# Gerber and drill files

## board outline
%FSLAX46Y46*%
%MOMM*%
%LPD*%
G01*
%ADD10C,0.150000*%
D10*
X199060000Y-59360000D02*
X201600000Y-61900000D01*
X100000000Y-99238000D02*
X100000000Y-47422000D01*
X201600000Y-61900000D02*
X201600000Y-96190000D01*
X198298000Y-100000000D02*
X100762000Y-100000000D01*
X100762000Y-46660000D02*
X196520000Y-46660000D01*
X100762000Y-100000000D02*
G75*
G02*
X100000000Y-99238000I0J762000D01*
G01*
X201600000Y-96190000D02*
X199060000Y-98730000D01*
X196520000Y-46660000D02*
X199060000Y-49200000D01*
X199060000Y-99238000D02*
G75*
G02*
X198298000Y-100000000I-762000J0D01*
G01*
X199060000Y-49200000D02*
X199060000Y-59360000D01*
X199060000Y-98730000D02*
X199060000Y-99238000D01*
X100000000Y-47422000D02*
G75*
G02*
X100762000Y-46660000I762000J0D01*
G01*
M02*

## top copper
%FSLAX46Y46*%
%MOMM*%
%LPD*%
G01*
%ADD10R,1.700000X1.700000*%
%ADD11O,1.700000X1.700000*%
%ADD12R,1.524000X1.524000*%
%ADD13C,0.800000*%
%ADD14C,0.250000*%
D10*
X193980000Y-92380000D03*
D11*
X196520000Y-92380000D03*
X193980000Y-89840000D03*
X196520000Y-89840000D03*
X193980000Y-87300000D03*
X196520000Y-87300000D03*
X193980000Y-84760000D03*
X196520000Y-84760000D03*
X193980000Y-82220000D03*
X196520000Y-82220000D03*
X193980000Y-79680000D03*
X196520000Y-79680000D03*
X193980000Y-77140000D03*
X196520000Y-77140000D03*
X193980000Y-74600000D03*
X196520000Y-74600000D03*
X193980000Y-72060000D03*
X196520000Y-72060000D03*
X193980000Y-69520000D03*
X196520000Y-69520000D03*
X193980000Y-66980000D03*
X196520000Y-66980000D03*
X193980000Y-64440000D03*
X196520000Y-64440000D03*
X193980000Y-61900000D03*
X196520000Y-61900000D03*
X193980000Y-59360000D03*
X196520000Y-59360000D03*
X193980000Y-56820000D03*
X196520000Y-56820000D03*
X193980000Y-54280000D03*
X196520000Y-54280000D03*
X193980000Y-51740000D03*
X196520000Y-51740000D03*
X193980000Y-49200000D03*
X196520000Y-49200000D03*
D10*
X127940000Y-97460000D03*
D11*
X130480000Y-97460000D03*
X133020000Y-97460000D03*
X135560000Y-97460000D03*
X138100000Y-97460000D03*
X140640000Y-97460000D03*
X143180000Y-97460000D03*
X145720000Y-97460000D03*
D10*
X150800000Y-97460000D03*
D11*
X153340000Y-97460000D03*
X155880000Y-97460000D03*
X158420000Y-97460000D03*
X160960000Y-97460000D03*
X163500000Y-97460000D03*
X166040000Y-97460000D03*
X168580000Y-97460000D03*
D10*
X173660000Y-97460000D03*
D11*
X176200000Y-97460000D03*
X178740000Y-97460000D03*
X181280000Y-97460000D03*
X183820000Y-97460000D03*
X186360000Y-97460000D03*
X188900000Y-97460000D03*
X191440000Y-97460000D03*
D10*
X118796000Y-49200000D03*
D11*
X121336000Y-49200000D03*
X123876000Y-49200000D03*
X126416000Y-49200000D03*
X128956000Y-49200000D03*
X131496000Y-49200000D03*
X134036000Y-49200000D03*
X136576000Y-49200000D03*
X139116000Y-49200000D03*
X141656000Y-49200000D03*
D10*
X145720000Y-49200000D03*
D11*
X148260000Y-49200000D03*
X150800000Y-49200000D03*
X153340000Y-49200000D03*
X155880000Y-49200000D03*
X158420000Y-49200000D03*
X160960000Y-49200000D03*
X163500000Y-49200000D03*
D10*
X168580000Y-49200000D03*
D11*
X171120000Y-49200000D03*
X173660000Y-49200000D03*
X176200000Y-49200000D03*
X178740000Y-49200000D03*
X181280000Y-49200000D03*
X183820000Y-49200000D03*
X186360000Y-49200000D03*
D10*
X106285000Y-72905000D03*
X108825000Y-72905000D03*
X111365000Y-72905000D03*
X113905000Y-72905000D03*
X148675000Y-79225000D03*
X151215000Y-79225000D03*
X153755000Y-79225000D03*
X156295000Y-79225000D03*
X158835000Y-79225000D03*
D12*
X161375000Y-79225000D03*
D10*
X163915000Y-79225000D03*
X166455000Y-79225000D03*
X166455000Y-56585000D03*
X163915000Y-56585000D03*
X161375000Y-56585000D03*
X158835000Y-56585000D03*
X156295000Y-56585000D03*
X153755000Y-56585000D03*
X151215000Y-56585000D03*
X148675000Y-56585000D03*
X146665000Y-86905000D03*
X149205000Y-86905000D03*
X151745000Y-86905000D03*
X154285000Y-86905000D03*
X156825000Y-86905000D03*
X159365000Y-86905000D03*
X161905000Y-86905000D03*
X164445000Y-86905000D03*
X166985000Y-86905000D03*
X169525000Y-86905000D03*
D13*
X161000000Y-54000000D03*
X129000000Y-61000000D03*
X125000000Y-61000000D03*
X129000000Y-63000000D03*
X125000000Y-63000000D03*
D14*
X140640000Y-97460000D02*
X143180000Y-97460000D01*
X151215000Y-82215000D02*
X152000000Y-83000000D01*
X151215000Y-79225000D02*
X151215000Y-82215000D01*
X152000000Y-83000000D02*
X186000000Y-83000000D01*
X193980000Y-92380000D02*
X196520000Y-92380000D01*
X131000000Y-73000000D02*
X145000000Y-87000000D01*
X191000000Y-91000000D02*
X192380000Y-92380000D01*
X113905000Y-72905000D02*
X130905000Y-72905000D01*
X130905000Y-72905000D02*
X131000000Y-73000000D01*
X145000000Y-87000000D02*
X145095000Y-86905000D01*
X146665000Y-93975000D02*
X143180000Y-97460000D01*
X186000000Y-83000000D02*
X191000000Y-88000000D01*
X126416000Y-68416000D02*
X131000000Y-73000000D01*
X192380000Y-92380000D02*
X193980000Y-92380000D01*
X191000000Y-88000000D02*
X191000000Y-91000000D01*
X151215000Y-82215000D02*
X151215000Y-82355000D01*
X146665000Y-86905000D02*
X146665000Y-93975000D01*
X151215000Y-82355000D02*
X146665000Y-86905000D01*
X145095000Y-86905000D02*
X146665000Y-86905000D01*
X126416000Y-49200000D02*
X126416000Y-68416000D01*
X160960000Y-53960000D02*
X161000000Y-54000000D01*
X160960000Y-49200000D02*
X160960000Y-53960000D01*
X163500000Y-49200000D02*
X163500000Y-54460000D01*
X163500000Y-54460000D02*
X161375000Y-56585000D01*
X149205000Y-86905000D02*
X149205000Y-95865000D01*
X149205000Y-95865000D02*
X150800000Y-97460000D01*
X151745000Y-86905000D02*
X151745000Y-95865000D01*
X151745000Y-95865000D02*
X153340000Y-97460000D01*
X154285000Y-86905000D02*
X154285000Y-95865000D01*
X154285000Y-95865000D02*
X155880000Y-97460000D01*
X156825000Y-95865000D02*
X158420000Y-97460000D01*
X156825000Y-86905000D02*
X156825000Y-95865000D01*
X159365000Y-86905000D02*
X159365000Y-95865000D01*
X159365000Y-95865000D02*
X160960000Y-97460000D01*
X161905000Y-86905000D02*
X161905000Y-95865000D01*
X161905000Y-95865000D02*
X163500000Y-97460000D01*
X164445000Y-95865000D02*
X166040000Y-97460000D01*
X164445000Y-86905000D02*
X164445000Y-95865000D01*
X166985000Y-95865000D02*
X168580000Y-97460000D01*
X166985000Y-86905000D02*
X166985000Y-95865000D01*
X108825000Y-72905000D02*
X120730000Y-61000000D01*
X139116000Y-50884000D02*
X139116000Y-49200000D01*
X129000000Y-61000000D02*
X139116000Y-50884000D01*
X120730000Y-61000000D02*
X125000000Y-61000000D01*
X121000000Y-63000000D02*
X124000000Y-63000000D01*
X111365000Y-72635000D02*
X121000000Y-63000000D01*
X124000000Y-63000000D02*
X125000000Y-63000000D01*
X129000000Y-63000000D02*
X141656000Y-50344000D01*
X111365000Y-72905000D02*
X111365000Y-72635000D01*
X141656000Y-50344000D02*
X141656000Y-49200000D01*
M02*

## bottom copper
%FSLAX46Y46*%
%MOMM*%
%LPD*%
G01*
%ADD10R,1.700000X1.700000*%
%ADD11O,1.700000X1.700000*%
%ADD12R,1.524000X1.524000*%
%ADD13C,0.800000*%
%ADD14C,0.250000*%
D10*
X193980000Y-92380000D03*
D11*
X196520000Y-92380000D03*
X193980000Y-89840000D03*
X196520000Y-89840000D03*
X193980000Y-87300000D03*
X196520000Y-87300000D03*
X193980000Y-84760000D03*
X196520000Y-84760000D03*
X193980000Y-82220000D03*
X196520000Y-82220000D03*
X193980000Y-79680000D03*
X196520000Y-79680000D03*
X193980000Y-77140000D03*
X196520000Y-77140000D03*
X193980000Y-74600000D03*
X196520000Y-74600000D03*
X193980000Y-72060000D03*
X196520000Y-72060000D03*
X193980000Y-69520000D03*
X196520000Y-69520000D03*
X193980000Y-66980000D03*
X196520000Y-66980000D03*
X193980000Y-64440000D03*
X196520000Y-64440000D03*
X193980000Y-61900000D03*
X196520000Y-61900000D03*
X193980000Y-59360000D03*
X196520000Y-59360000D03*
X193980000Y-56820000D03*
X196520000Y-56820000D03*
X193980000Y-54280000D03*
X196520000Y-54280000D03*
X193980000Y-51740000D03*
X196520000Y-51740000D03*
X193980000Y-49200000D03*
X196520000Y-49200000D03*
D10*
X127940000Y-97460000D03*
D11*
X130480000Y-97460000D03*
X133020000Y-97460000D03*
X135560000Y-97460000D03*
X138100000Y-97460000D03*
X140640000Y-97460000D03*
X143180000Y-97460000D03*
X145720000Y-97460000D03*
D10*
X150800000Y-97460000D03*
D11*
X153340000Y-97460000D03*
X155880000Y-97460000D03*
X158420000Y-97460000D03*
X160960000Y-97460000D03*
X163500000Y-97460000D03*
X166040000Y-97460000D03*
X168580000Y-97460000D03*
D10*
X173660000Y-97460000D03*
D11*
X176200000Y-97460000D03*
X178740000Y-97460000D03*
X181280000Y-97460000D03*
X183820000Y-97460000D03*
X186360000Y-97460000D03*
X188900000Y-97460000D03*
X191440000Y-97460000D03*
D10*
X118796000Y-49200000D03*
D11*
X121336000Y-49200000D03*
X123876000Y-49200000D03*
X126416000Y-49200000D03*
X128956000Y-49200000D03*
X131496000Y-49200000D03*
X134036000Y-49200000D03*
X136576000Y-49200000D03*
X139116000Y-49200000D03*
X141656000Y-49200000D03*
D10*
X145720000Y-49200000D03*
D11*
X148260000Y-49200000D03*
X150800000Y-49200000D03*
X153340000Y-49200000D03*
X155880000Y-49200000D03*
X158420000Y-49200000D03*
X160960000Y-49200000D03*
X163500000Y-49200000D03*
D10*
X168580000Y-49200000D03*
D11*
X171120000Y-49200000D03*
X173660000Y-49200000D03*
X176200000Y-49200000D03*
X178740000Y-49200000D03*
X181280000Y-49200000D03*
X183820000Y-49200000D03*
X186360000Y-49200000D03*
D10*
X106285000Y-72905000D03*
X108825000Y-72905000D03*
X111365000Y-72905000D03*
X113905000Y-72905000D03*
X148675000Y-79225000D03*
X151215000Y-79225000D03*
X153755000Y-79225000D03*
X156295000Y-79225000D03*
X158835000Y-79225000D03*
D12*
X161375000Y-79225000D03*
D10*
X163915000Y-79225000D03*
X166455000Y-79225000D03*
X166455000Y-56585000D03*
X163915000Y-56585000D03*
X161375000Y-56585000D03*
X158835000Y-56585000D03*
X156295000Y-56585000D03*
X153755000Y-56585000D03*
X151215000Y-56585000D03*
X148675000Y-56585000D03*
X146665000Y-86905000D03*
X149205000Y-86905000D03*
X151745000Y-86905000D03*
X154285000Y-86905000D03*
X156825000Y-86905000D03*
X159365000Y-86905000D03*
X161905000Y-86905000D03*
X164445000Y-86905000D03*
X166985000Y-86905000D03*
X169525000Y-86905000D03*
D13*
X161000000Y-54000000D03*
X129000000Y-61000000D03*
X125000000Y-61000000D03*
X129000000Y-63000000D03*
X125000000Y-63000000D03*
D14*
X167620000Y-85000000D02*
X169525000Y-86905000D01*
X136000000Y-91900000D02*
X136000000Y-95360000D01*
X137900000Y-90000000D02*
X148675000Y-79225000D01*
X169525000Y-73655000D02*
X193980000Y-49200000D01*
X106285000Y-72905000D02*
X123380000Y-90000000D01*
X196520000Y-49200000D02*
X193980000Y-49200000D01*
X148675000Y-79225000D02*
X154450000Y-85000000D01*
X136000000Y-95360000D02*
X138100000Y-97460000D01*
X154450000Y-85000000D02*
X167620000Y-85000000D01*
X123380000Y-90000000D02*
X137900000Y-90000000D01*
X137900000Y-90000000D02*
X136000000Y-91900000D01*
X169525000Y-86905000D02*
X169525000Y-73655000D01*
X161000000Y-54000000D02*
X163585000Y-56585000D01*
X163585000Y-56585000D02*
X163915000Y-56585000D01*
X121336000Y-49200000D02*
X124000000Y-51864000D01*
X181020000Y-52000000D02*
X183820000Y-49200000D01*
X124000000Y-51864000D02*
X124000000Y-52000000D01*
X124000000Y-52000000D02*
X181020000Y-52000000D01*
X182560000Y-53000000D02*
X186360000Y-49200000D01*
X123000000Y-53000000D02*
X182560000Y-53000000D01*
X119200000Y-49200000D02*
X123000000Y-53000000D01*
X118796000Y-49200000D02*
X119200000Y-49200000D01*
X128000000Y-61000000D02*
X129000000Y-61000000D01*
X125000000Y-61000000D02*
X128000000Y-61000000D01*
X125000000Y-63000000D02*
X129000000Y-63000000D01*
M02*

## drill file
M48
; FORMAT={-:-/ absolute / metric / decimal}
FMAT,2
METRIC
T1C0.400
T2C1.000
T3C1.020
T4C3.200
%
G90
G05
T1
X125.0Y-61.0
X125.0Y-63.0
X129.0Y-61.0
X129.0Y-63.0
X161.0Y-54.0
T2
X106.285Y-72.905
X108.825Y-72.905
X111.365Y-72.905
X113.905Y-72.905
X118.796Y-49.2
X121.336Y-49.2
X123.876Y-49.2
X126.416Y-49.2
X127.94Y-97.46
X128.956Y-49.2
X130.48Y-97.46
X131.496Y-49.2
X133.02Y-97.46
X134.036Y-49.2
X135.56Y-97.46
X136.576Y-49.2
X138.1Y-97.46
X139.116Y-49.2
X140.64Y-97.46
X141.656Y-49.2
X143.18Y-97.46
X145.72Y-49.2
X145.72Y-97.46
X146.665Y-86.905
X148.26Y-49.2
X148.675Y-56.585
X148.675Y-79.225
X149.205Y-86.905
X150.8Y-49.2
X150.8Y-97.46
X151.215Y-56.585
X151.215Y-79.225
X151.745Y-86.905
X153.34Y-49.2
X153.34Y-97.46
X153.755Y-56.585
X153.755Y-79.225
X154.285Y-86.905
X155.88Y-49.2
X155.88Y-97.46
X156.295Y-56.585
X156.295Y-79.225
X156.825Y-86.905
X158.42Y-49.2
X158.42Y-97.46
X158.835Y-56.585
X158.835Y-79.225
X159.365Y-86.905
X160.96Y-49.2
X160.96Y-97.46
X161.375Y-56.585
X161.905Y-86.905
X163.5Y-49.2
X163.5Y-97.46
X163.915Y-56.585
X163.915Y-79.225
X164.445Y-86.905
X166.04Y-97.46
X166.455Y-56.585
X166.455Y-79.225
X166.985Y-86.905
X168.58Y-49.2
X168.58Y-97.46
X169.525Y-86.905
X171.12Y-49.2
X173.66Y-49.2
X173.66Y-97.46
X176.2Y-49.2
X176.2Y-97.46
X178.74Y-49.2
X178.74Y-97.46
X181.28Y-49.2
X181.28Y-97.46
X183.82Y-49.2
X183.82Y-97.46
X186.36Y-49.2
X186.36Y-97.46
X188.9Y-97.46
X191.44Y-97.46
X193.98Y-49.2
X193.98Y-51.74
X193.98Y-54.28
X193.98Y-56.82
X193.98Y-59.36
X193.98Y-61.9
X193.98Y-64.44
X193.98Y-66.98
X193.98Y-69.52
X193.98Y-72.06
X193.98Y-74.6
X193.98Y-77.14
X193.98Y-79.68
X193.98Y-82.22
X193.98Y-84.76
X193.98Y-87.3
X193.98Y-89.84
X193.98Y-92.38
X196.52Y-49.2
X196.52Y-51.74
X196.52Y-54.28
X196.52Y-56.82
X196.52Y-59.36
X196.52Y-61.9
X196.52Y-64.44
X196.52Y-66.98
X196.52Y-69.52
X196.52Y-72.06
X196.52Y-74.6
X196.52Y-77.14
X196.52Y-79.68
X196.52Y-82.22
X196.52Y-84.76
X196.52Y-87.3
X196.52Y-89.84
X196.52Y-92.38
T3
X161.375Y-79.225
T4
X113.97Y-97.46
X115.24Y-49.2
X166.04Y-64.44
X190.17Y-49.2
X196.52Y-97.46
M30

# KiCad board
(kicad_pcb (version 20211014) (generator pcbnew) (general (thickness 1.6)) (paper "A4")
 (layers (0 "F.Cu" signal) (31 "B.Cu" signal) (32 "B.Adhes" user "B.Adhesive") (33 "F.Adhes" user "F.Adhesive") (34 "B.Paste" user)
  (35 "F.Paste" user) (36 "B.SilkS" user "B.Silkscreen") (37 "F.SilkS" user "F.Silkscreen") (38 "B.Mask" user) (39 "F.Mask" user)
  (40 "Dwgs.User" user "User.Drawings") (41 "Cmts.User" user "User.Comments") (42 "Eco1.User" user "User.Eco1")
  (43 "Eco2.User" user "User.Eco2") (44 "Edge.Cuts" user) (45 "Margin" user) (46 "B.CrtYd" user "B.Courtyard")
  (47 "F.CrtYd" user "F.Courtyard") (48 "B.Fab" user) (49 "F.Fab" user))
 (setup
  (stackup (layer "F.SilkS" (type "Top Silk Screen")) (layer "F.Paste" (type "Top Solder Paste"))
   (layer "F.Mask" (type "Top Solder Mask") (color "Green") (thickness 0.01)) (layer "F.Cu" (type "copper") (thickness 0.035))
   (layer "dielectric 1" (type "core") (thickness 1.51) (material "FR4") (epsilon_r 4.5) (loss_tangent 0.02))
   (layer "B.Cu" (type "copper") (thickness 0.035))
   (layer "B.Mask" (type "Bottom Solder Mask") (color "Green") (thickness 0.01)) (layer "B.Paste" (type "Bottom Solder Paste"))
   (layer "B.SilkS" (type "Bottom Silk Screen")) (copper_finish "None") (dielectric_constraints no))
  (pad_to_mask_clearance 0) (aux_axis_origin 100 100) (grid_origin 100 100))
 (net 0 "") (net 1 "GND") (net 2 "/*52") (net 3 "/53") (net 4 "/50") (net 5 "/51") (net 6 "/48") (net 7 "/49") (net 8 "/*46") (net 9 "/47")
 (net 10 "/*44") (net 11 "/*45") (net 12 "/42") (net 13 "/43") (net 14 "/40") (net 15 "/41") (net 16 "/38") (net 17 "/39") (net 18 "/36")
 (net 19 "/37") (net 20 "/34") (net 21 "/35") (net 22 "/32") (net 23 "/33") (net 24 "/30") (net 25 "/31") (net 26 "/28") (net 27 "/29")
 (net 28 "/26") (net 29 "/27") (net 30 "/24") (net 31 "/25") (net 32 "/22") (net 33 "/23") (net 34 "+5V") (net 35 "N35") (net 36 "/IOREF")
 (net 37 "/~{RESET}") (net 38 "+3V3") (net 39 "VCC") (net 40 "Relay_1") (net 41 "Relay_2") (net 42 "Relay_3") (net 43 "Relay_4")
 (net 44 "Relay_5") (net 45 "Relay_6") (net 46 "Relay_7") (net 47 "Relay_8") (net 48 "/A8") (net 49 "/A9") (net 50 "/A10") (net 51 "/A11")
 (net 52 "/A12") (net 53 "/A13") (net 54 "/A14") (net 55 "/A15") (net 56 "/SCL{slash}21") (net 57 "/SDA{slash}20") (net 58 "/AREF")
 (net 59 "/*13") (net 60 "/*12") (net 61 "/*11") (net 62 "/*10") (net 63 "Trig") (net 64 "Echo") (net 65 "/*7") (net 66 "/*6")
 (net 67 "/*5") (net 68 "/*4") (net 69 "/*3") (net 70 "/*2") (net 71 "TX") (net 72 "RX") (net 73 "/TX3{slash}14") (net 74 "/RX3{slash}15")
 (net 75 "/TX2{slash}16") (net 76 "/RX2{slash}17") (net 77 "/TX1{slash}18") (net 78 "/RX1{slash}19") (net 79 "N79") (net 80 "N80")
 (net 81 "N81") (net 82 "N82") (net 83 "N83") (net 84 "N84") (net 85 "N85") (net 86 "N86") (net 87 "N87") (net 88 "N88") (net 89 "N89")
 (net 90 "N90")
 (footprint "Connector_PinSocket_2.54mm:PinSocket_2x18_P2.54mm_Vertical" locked (layer "F.Cu") (at 193.98 92.38 180)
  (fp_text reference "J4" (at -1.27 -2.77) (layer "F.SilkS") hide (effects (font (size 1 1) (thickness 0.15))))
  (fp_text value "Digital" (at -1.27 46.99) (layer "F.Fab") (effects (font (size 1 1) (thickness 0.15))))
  (pad "1" thru_hole rect locked (at 0 0 180) (size 1.7 1.7) (drill 1) (layers *.Cu *.Mask) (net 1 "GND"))
  (pad "2" thru_hole oval locked (at -2.54 0 180) (size 1.7 1.7) (drill 1) (layers *.Cu *.Mask) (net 1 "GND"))
  (pad "3" thru_hole oval locked (at 0 2.54 180) (size 1.7 1.7) (drill 1) (layers *.Cu *.Mask) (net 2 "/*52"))
  (pad "4" thru_hole oval locked (at -2.54 2.54 180) (size 1.7 1.7) (drill 1) (layers *.Cu *.Mask) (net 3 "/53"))
  (pad "5" thru_hole oval locked (at 0 5.08 180) (size 1.7 1.7) (drill 1) (layers *.Cu *.Mask) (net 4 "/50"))
  (pad "6" thru_hole oval locked (at -2.54 5.08 180) (size 1.7 1.7) (drill 1) (layers *.Cu *.Mask) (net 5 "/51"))
  (pad "7" thru_hole oval locked (at 0 7.62 180) (size 1.7 1.7) (drill 1) (layers *.Cu *.Mask) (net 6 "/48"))
  (pad "8" thru_hole oval locked (at -2.54 7.62 180) (size 1.7 1.7) (drill 1) (layers *.Cu *.Mask) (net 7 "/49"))
  (pad "9" thru_hole oval locked (at 0 10.16 180) (size 1.7 1.7) (drill 1) (layers *.Cu *.Mask) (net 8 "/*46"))
  (pad "10" thru_hole oval locked (at -2.54 10.16 180) (size 1.7 1.7) (drill 1) (layers *.Cu *.Mask) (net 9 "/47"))
  (pad "11" thru_hole oval locked (at 0 12.7 180) (size 1.7 1.7) (drill 1) (layers *.Cu *.Mask) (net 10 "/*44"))
  (pad "12" thru_hole oval locked (at -2.54 12.7 180) (size 1.7 1.7) (drill 1) (layers *.Cu *.Mask) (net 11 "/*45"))
  (pad "13" thru_hole oval locked (at 0 15.24 180) (size 1.7 1.7) (drill 1) (layers *.Cu *.Mask) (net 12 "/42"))
  (pad "14" thru_hole oval locked (at -2.54 15.24 180) (size 1.7 1.7) (drill 1) (layers *.Cu *.Mask) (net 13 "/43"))
  (pad "15" thru_hole oval locked (at 0 17.78 180) (size 1.7 1.7) (drill 1) (layers *.Cu *.Mask) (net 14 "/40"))
  (pad "16" thru_hole oval locked (at -2.54 17.78 180) (size 1.7 1.7) (drill 1) (layers *.Cu *.Mask) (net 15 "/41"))
  (pad "17" thru_hole oval locked (at 0 20.32 180) (size 1.7 1.7) (drill 1) (layers *.Cu *.Mask) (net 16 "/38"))
  (pad "18" thru_hole oval locked (at -2.54 20.32 180) (size 1.7 1.7) (drill 1) (layers *.Cu *.Mask) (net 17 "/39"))
  (pad "19" thru_hole oval locked (at 0 22.86 180) (size 1.7 1.7) (drill 1) (layers *.Cu *.Mask) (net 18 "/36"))
  (pad "20" thru_hole oval locked (at -2.54 22.86 180) (size 1.7 1.7) (drill 1) (layers *.Cu *.Mask) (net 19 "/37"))
  (pad "21" thru_hole oval locked (at 0 25.4 180) (size 1.7 1.7) (drill 1) (layers *.Cu *.Mask) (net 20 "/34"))
  (pad "22" thru_hole oval locked (at -2.54 25.4 180) (size 1.7 1.7) (drill 1) (layers *.Cu *.Mask) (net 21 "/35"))
  (pad "23" thru_hole oval locked (at 0 27.94 180) (size 1.7 1.7) (drill 1) (layers *.Cu *.Mask) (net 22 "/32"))
  (pad "24" thru_hole oval locked (at -2.54 27.94 180) (size 1.7 1.7) (drill 1) (layers *.Cu *.Mask) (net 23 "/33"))
  (pad "25" thru_hole oval locked (at 0 30.48 180) (size 1.7 1.7) (drill 1) (layers *.Cu *.Mask) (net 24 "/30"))
  (pad "26" thru_hole oval locked (at -2.54 30.48 180) (size 1.7 1.7) (drill 1) (layers *.Cu *.Mask) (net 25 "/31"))
  (pad "27" thru_hole oval locked (at 0 33.02 180) (size 1.7 1.7) (drill 1) (layers *.Cu *.Mask) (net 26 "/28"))
  (pad "28" thru_hole oval locked (at -2.54 33.02 180) (size 1.7 1.7) (drill 1) (layers *.Cu *.Mask) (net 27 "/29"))
  (pad "29" thru_hole oval locked (at 0 35.56 180) (size 1.7 1.7) (drill 1) (layers *.Cu *.Mask) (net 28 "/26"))
  (pad "30" thru_hole oval locked (at -2.54 35.56 180) (size 1.7 1.7) (drill 1) (layers *.Cu *.Mask) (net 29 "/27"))
  (pad "31" thru_hole oval locked (at 0 38.1 180) (size 1.7 1.7) (drill 1) (layers *.Cu *.Mask) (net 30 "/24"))
  (pad "32" thru_hole oval locked (at -2.54 38.1 180) (size 1.7 1.7) (drill 1) (layers *.Cu *.Mask) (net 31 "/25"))
  (pad "33" thru_hole oval locked (at 0 40.64 180) (size 1.7 1.7) (drill 1) (layers *.Cu *.Mask) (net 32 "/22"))
  (pad "34" thru_hole oval locked (at -2.54 40.64 180) (size 1.7 1.7) (drill 1) (layers *.Cu *.Mask) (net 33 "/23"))
  (pad "35" thru_hole oval locked (at 0 43.18 180) (size 1.7 1.7) (drill 1) (layers *.Cu *.Mask) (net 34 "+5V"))
  (pad "36" thru_hole oval locked (at -2.54 43.18 180) (size 1.7 1.7) (drill 1) (layers *.Cu *.Mask) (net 34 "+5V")))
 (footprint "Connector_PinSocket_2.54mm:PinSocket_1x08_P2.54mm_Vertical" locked (layer "F.Cu") (at 127.94 97.46 90)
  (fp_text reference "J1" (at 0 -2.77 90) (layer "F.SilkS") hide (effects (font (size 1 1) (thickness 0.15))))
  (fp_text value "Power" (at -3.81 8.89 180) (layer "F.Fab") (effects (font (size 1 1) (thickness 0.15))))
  (pad "1" thru_hole rect locked (at 0 0 90) (size 1.7 1.7) (drill 1) (layers *.Cu *.Mask) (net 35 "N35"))
  (pad "2" thru_hole oval locked (at 0 2.54 90) (size 1.7 1.7) (drill 1) (layers *.Cu *.Mask) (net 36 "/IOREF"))
  (pad "3" thru_hole oval locked (at 0 5.08 90) (size 1.7 1.7) (drill 1) (layers *.Cu *.Mask) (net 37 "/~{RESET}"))
  (pad "4" thru_hole oval locked (at 0 7.62 90) (size 1.7 1.7) (drill 1) (layers *.Cu *.Mask) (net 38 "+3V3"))
  (pad "5" thru_hole oval locked (at 0 10.16 90) (size 1.7 1.7) (drill 1) (layers *.Cu *.Mask) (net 34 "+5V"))
  (pad "6" thru_hole oval locked (at 0 12.7 90) (size 1.7 1.7) (drill 1) (layers *.Cu *.Mask) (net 1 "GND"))
  (pad "7" thru_hole oval locked (at 0 15.24 90) (size 1.7 1.7) (drill 1) (layers *.Cu *.Mask) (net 1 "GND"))
  (pad "8" thru_hole oval locked (at 0 17.78 90) (size 1.7 1.7) (drill 1) (layers *.Cu *.Mask) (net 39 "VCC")))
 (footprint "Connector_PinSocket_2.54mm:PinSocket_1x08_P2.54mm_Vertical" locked (layer "F.Cu") (at 150.8 97.46 90)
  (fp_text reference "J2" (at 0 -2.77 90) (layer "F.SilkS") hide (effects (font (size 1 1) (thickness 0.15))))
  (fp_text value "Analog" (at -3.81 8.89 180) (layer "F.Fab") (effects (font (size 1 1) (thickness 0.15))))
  (pad "1" thru_hole rect locked (at 0 0 90) (size 1.7 1.7) (drill 1) (layers *.Cu *.Mask) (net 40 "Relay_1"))
  (pad "2" thru_hole oval locked (at 0 2.54 90) (size 1.7 1.7) (drill 1) (layers *.Cu *.Mask) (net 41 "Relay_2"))
  (pad "3" thru_hole oval locked (at 0 5.08 90) (size 1.7 1.7) (drill 1) (layers *.Cu *.Mask) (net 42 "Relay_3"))
  (pad "4" thru_hole oval locked (at 0 7.62 90) (size 1.7 1.7) (drill 1) (layers *.Cu *.Mask) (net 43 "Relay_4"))
  (pad "5" thru_hole oval locked (at 0 10.16 90) (size 1.7 1.7) (drill 1) (layers *.Cu *.Mask) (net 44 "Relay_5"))
  (pad "6" thru_hole oval locked (at 0 12.7 90) (size 1.7 1.7) (drill 1) (layers *.Cu *.Mask) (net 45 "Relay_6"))
  (pad "7" thru_hole oval locked (at 0 15.24 90) (size 1.7 1.7) (drill 1) (layers *.Cu *.Mask) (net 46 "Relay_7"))
  (pad "8" thru_hole oval locked (at 0 17.78 90) (size 1.7 1.7) (drill 1) (layers *.Cu *.Mask) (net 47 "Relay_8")))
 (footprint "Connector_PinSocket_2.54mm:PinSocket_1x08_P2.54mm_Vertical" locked (layer "F.Cu") (at 173.66 97.46 90)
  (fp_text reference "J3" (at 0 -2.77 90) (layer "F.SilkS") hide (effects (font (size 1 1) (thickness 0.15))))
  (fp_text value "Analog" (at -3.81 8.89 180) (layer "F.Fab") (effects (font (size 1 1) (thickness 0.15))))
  (pad "1" thru_hole rect locked (at 0 0 90) (size 1.7 1.7) (drill 1) (layers *.Cu *.Mask) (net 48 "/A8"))
  (pad "2" thru_hole oval locked (at 0 2.54 90) (size 1.7 1.7) (drill 1) (layers *.Cu *.Mask) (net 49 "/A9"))
  (pad "3" thru_hole oval locked (at 0 5.08 90) (size 1.7 1.7) (drill 1) (layers *.Cu *.Mask) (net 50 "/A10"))
  (pad "4" thru_hole oval locked (at 0 7.62 90) (size 1.7 1.7) (drill 1) (layers *.Cu *.Mask) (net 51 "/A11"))
  (pad "5" thru_hole oval locked (at 0 10.16 90) (size 1.7 1.7) (drill 1) (layers *.Cu *.Mask) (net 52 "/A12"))
  (pad "6" thru_hole oval locked (at 0 12.7 90) (size 1.7 1.7) (drill 1) (layers *.Cu *.Mask) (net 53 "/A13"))
  (pad "7" thru_hole oval locked (at 0 15.24 90) (size 1.7 1.7) (drill 1) (layers *.Cu *.Mask) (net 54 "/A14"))
  (pad "8" thru_hole oval locked (at 0 17.78 90) (size 1.7 1.7) (drill 1) (layers *.Cu *.Mask) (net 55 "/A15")))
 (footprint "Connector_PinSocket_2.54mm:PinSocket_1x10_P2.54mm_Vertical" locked (layer "F.Cu") (at 118.796 49.2 90)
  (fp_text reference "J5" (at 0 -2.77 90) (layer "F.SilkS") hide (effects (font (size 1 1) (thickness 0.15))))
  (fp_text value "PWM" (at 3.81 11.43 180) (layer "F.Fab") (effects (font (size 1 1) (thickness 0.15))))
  (pad "1" thru_hole rect locked (at 0 0 90) (size 1.7 1.7) (drill 1) (layers *.Cu *.Mask) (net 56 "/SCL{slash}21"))
  (pad "2" thru_hole oval locked (at 0 2.54 90) (size 1.7 1.7) (drill 1) (layers *.Cu *.Mask) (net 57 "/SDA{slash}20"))
  (pad "3" thru_hole oval locked (at 0 5.08 90) (size 1.7 1.7) (drill 1) (layers *.Cu *.Mask) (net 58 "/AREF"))
  (pad "4" thru_hole oval locked (at 0 7.62 90) (size 1.7 1.7) (drill 1) (layers *.Cu *.Mask) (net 1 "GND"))
  (pad "5" thru_hole oval locked (at 0 10.16 90) (size 1.7 1.7) (drill 1) (layers *.Cu *.Mask) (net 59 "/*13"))
  (pad "6" thru_hole oval locked (at 0 12.7 90) (size 1.7 1.7) (drill 1) (layers *.Cu *.Mask) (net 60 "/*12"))
  (pad "7" thru_hole oval locked (at 0 15.24 90) (size 1.7 1.7) (drill 1) (layers *.Cu *.Mask) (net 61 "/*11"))
  (pad "8" thru_hole oval locked (at 0 17.78 90) (size 1.7 1.7) (drill 1) (layers *.Cu *.Mask) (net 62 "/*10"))
  (pad "9" thru_hole oval locked (at 0 20.32 90) (size 1.7 1.7) (drill 1) (layers *.Cu *.Mask) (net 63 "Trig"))
  (pad "10" thru_hole oval locked (at 0 22.86 90) (size 1.7 1.7) (drill 1) (layers *.Cu *.Mask) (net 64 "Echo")))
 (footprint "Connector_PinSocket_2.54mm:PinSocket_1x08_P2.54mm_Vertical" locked (layer "F.Cu") (at 145.72 49.2 90)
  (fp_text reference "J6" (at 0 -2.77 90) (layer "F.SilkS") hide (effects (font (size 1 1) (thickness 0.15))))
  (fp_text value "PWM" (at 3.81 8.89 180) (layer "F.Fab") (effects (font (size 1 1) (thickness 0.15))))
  (pad "1" thru_hole rect locked (at 0 0 90) (size 1.7 1.7) (drill 1) (layers *.Cu *.Mask) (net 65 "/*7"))
  (pad "2" thru_hole oval locked (at 0 2.54 90) (size 1.7 1.7) (drill 1) (layers *.Cu *.Mask) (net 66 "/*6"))
  (pad "3" thru_hole oval locked (at 0 5.08 90) (size 1.7 1.7) (drill 1) (layers *.Cu *.Mask) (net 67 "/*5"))
  (pad "4" thru_hole oval locked (at 0 7.62 90) (size 1.7 1.7) (drill 1) (layers *.Cu *.Mask) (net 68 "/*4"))
  (pad "5" thru_hole oval locked (at 0 10.16 90) (size 1.7 1.7) (drill 1) (layers *.Cu *.Mask) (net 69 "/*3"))
  (pad "6" thru_hole oval locked (at 0 12.7 90) (size 1.7 1.7) (drill 1) (layers *.Cu *.Mask) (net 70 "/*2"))
  (pad "7" thru_hole oval locked (at 0 15.24 90) (size 1.7 1.7) (drill 1) (layers *.Cu *.Mask) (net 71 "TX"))
  (pad "8" thru_hole oval locked (at 0 17.78 90) (size 1.7 1.7) (drill 1) (layers *.Cu *.Mask) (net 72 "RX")))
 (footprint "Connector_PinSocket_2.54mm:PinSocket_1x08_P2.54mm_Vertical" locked (layer "F.Cu") (at 168.58 49.2 90)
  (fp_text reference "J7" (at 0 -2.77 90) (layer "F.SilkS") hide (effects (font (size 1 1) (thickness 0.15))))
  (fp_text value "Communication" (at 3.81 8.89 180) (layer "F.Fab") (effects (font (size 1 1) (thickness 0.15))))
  (pad "1" thru_hole rect locked (at 0 0 90) (size 1.7 1.7) (drill 1) (layers *.Cu *.Mask) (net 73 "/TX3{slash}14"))
  (pad "2" thru_hole oval locked (at 0 2.54 90) (size 1.7 1.7) (drill 1) (layers *.Cu *.Mask) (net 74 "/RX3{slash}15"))
  (pad "3" thru_hole oval locked (at 0 5.08 90) (size 1.7 1.7) (drill 1) (layers *.Cu *.Mask) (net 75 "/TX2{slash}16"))
  (pad "4" thru_hole oval locked (at 0 7.62 90) (size 1.7 1.7) (drill 1) (layers *.Cu *.Mask) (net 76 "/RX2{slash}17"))
  (pad "5" thru_hole oval locked (at 0 10.16 90) (size 1.7 1.7) (drill 1) (layers *.Cu *.Mask) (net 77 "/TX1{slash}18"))
  (pad "6" thru_hole oval locked (at 0 12.7 90) (size 1.7 1.7) (drill 1) (layers *.Cu *.Mask) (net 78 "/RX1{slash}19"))
  (pad "7" thru_hole oval locked (at 0 15.24 90) (size 1.7 1.7) (drill 1) (layers *.Cu *.Mask) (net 57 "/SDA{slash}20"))
  (pad "8" thru_hole oval locked (at 0 17.78 90) (size 1.7 1.7) (drill 1) (layers *.Cu *.Mask) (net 56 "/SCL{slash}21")))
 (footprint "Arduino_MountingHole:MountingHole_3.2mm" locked (layer "F.Cu") (at 196.52 97.46)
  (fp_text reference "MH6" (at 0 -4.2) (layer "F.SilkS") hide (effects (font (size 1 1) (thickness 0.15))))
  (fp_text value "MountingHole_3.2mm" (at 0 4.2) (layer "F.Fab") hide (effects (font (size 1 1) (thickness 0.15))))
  (pad "" np_thru_hole circle locked (at 0 0) (size 3.2 3.2) (drill 3.2) (layers *.Cu *.Mask)))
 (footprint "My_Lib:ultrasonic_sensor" (layer "F.Cu") (at 103.745 75.445 90)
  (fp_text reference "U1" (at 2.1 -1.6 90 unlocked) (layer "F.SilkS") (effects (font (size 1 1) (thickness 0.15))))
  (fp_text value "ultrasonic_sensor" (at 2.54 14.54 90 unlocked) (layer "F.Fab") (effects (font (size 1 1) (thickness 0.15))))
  (pad "1" thru_hole rect (at 2.54 2.54 90) (size 1.7 1.7) (drill 1) (layers *.Cu *.Mask) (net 34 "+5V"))
  (pad "2" thru_hole rect (at 2.54 5.08 90) (size 1.7 1.7) (drill 1) (layers *.Cu *.Mask) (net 63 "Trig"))
  (pad "3" thru_hole rect (at 2.54 7.62 90) (size 1.7 1.7) (drill 1) (layers *.Cu *.Mask) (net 64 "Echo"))
  (pad "4" thru_hole rect (at 2.54 10.16 90) (size 1.7 1.7) (drill 1) (layers *.Cu *.Mask) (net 1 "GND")))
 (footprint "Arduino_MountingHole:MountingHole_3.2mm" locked (layer "F.Cu") (at 115.24 49.2)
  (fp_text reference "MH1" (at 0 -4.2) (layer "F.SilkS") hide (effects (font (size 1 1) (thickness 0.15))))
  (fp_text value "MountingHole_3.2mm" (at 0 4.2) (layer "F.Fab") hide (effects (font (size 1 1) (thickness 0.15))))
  (pad "" np_thru_hole circle locked (at 0 0) (size 3.2 3.2) (drill 3.2) (layers *.Cu *.Mask)))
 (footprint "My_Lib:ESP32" (layer "F.Cu") (at 144.095 81.405 90)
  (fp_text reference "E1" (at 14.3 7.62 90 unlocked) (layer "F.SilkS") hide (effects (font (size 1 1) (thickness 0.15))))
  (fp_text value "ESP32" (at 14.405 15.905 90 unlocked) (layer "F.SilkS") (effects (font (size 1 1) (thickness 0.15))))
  (pad "1" thru_hole rect (at 2.18 4.58 270) (size 1.7 1.7) (drill 1) (layers *.Cu *.Mask) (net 34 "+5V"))
  (pad "2" thru_hole rect (at 2.18 7.12 270) (size 1.7 1.7) (drill 1) (layers *.Cu *.Mask) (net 1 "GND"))
  (pad "3" thru_hole rect (at 2.18 9.66 270) (size 1.7 1.7) (drill 1) (layers *.Cu *.Mask) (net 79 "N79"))
  (pad "4" thru_hole rect (at 2.18 12.2 270) (size 1.7 1.7) (drill 1) (layers *.Cu *.Mask) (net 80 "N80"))
  (pad "5" thru_hole rect (at 2.18 14.74 270) (size 1.7 1.7) (drill 1) (layers *.Cu *.Mask) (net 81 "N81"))
  (pad "6" thru_hole rect (at 2.18 17.28 270) (size 1.524 1.524) (drill 1.02) (layers *.Cu *.Mask) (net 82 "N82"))
  (pad "7" thru_hole rect (at 2.18 19.82 270) (size 1.7 1.7) (drill 1) (layers *.Cu *.Mask) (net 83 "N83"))
  (pad "8" thru_hole rect (at 2.18 22.36 270) (size 1.7 1.7) (drill 1) (layers *.Cu *.Mask) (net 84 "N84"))
  (pad "9" thru_hole rect (at 24.82 22.36 270) (size 1.7 1.7) (drill 1) (layers *.Cu *.Mask) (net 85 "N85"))
  (pad "10" thru_hole rect (at 24.82 19.82 270) (size 1.7 1.7) (drill 1) (layers *.Cu *.Mask) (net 71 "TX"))
  (pad "11" thru_hole rect (at 24.82 17.28 270) (size 1.7 1.7) (drill 1) (layers *.Cu *.Mask) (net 72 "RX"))
  (pad "12" thru_hole rect (at 24.82 14.74 270) (size 1.7 1.7) (drill 1) (layers *.Cu *.Mask) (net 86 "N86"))
  (pad "13" thru_hole rect (at 24.82 12.2 270) (size 1.7 1.7) (drill 1) (layers *.Cu *.Mask) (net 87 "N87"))
  (pad "14" thru_hole rect (at 24.82 9.66 270) (size 1.7 1.7) (drill 1) (layers *.Cu *.Mask) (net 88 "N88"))
  (pad "15" thru_hole rect (at 24.82 7.12 270) (size 1.7 1.7) (drill 1) (layers *.Cu *.Mask) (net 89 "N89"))
  (pad "16" thru_hole rect (at 24.82 4.58 270) (size 1.7 1.7) (drill 1) (layers *.Cu *.Mask) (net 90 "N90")))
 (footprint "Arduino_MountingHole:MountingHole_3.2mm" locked (layer "F.Cu") (at 113.97 97.46)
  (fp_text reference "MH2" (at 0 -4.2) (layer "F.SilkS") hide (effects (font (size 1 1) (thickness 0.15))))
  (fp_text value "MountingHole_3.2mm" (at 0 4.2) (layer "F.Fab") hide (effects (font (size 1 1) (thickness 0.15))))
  (pad "" np_thru_hole circle locked (at 0 0) (size 3.2 3.2) (drill 3.2) (layers *.Cu *.Mask)))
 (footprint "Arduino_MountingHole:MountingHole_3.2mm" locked (layer "F.Cu") (at 166.04 64.44)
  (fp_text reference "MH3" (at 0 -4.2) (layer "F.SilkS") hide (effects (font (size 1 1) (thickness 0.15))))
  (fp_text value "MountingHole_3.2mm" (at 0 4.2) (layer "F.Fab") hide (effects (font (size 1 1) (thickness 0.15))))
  (pad "" np_thru_hole circle locked (at 0 0) (size 3.2 3.2) (drill 3.2) (layers *.Cu *.Mask)))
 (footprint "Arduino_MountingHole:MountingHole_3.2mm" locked (layer "F.Cu") (at 190.17 49.2)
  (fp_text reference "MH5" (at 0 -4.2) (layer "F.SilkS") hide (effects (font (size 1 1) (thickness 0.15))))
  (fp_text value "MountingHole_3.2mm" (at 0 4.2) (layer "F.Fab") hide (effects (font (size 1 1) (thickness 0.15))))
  (pad "" np_thru_hole circle locked (at 0 0) (size 3.2 3.2) (drill 3.2) (layers *.Cu *.Mask)))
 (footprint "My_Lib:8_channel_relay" (layer "F.Cu") (at 144.125 89.445 90)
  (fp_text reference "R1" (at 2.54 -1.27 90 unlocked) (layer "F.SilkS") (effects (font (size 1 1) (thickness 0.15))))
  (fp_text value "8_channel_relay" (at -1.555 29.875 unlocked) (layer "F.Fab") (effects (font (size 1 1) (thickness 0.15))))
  (pad "1" thru_hole rect (at 2.54 2.54 90) (size 1.7 1.7) (drill 1) (layers *.Cu *.Mask) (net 1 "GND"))
  (pad "2" thru_hole rect (at 2.54 5.08 90) (size 1.7 1.7) (drill 1) (layers *.Cu *.Mask) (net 40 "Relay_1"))
  (pad "3" thru_hole rect (at 2.54 7.62 90) (size 1.7 1.7) (drill 1) (layers *.Cu *.Mask) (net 41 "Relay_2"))
  (pad "4" thru_hole rect (at 2.54 10.16 90) (size 1.7 1.7) (drill 1) (layers *.Cu *.Mask) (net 42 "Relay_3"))
  (pad "5" thru_hole rect (at 2.54 12.7 90) (size 1.7 1.7) (drill 1) (layers *.Cu *.Mask) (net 43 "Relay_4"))
  (pad "6" thru_hole rect (at 2.54 15.24 90) (size 1.7 1.7) (drill 1) (layers *.Cu *.Mask) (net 44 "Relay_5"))
  (pad "7" thru_hole rect (at 2.54 17.78 90) (size 1.7 1.7) (drill 1) (layers *.Cu *.Mask) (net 45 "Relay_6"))
  (pad "8" thru_hole rect (at 2.54 20.32 90) (size 1.7 1.7) (drill 1) (layers *.Cu *.Mask) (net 46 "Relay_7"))
  (pad "9" thru_hole rect (at 2.54 22.86 90) (size 1.7 1.7) (drill 1) (layers *.Cu *.Mask) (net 47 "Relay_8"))
  (pad "10" thru_hole rect (at 2.54 25.4 90) (size 1.7 1.7) (drill 1) (layers *.Cu *.Mask) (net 34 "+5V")))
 (gr_line (start 199.06 59.36) (end 201.6 61.9) (layer "Edge.Cuts") (width 0.15))
 (gr_line (start 100 99.238) (end 100 47.422) (layer "Edge.Cuts") (width 0.15))
 (gr_line (start 201.6 61.9) (end 201.6 96.19) (layer "Edge.Cuts") (width 0.15))
 (gr_line (start 198.298 100) (end 100.762 100) (layer "Edge.Cuts") (width 0.15))
 (gr_line (start 100.762 46.66) (end 196.52 46.66) (layer "Edge.Cuts") (width 0.15))
 (gr_arc (start 100.762 100) (mid 100.223185 99.776815) (end 100 99.238) (layer "Edge.Cuts") (width 0.15))
 (gr_line (start 201.6 96.19) (end 199.06 98.73) (layer "Edge.Cuts") (width 0.15))
 (gr_line (start 196.52 46.66) (end 199.06 49.2) (layer "Edge.Cuts") (width 0.15))
 (gr_arc (start 199.06 99.238) (mid 198.836815 99.776815) (end 198.298 100) (layer "Edge.Cuts") (width 0.15))
 (gr_line (start 199.06 49.2) (end 199.06 59.36) (layer "Edge.Cuts") (width 0.15))
 (gr_line (start 199.06 98.73) (end 199.06 99.238) (layer "Edge.Cuts") (width 0.15))
 (gr_arc (start 100 47.422) (mid 100.223185 46.883185) (end 100.762 46.66) (layer "Edge.Cuts") (width 0.15))
 (segment (start 140.64 97.46) (end 143.18 97.46) (width 0.25) (layer "F.Cu") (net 1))
 (segment (start 151.215 82.215) (end 152 83) (width 0.25) (layer "F.Cu") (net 1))
 (segment (start 151.215 79.225) (end 151.215 82.215) (width 0.25) (layer "F.Cu") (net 1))
 (segment (start 152 83) (end 186 83) (width 0.25) (layer "F.Cu") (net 1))
 (segment (start 193.98 92.38) (end 196.52 92.38) (width 0.25) (layer "F.Cu") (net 1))
 (segment (start 131 73) (end 145 87) (width 0.25) (layer "F.Cu") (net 1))
 (segment (start 191 91) (end 192.38 92.38) (width 0.25) (layer "F.Cu") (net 1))
 (segment (start 113.905 72.905) (end 130.905 72.905) (width 0.25) (layer "F.Cu") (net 1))
 (segment (start 130.905 72.905) (end 131 73) (width 0.25) (layer "F.Cu") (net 1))
 (segment (start 145 87) (end 145.095 86.905) (width 0.25) (layer "F.Cu") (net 1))
 (segment (start 146.665 93.975) (end 143.18 97.46) (width 0.25) (layer "F.Cu") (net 1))
 (segment (start 186 83) (end 191 88) (width 0.25) (layer "F.Cu") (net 1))
 (segment (start 126.416 68.416) (end 131 73) (width 0.25) (layer "F.Cu") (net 1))
 (segment (start 192.38 92.38) (end 193.98 92.38) (width 0.25) (layer "F.Cu") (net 1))
 (segment (start 191 88) (end 191 91) (width 0.25) (layer "F.Cu") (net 1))
 (segment (start 151.215 82.215) (end 151.215 82.355) (width 0.25) (layer "F.Cu") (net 1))
 (segment (start 146.665 86.905) (end 146.665 93.975) (width 0.25) (layer "F.Cu") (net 1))
 (segment (start 151.215 82.355) (end 146.665 86.905) (width 0.25) (layer "F.Cu") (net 1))
 (segment (start 145.095 86.905) (end 146.665 86.905) (width 0.25) (layer "F.Cu") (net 1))
 (segment (start 126.416 49.2) (end 126.416 68.416) (width 0.25) (layer "F.Cu") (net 1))
 (segment (start 167.62 85) (end 169.525 86.905) (width 0.25) (layer "B.Cu") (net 34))
 (segment (start 136 91.9) (end 136 95.36) (width 0.25) (layer "B.Cu") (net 34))
 (segment (start 137.9 90) (end 148.675 79.225) (width 0.25) (layer "B.Cu") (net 34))
 (segment (start 169.525 73.655) (end 193.98 49.2) (width 0.25) (layer "B.Cu") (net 34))
 (segment (start 106.285 72.905) (end 123.38 90) (width 0.25) (layer "B.Cu") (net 34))
 (segment (start 196.52 49.2) (end 193.98 49.2) (width 0.25) (layer "B.Cu") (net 34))
 (segment (start 148.675 79.225) (end 154.45 85) (width 0.25) (layer "B.Cu") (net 34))
 (segment (start 136 95.36) (end 138.1 97.46) (width 0.25) (layer "B.Cu") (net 34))
 (segment (start 154.45 85) (end 167.62 85) (width 0.25) (layer "B.Cu") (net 34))
 (segment (start 123.38 90) (end 137.9 90) (width 0.25) (layer "B.Cu") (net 34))
 (segment (start 137.9 90) (end 136 91.9) (width 0.25) (layer "B.Cu") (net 34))
 (segment (start 169.525 86.905) (end 169.525 73.655) (width 0.25) (layer "B.Cu") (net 34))
 (segment (start 160.96 53.96) (end 161 54) (width 0.25) (layer "F.Cu") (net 71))
 (segment (start 160.96 49.2) (end 160.96 53.96) (width 0.25) (layer "F.Cu") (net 71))
 (via (at 161 54) (size 0.8) (drill 0.4) (layers "F.Cu" "B.Cu") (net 71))
 (segment (start 161 54) (end 163.585 56.585) (width 0.25) (layer "B.Cu") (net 71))
 (segment (start 163.585 56.585) (end 163.915 56.585) (width 0.25) (layer "B.Cu") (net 71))
 (segment (start 163.5 49.2) (end 163.5 54.46) (width 0.25) (layer "F.Cu") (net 72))
 (segment (start 163.5 54.46) (end 161.375 56.585) (width 0.25) (layer "F.Cu") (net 72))
 (segment (start 121.336 49.2) (end 124 51.864) (width 0.25) (layer "B.Cu") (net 57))
 (segment (start 181.02 52) (end 183.82 49.2) (width 0.25) (layer "B.Cu") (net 57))
 (segment (start 124 51.864) (end 124 52) (width 0.25) (layer "B.Cu") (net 57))
 (segment (start 124 52) (end 181.02 52) (width 0.25) (layer "B.Cu") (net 57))
 (segment (start 182.56 53) (end 186.36 49.2) (width 0.25) (layer "B.Cu") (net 56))
 (segment (start 123 53) (end 182.56 53) (width 0.25) (layer "B.Cu") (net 56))
 (segment (start 119.2 49.2) (end 123 53) (width 0.25) (layer "B.Cu") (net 56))
 (segment (start 118.796 49.2) (end 119.2 49.2) (width 0.25) (layer "B.Cu") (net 56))
 (segment (start 149.205 86.905) (end 149.205 95.865) (width 0.25) (layer "F.Cu") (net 40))
 (segment (start 149.205 95.865) (end 150.8 97.46) (width 0.25) (layer "F.Cu") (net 40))
 (segment (start 151.745 86.905) (end 151.745 95.865) (width 0.25) (layer "F.Cu") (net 41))
 (segment (start 151.745 95.865) (end 153.34 97.46) (width 0.25) (layer "F.Cu") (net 41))
 (segment (start 154.285 86.905) (end 154.285 95.865) (width 0.25) (layer "F.Cu") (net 42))
 (segment (start 154.285 95.865) (end 155.88 97.46) (width 0.25) (layer "F.Cu") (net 42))
 (segment (start 156.825 95.865) (end 158.42 97.46) (width 0.25) (layer "F.Cu") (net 43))
 (segment (start 156.825 86.905) (end 156.825 95.865) (width 0.25) (layer "F.Cu") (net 43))
 (segment (start 159.365 86.905) (end 159.365 95.865) (width 0.25) (layer "F.Cu") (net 44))
 (segment (start 159.365 95.865) (end 160.96 97.46) (width 0.25) (layer "F.Cu") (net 44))
 (segment (start 161.905 86.905) (end 161.905 95.865) (width 0.25) (layer "F.Cu") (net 45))
 (segment (start 161.905 95.865) (end 163.5 97.46) (width 0.25) (layer "F.Cu") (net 45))
 (segment (start 164.445 95.865) (end 166.04 97.46) (width 0.25) (layer "F.Cu") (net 46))
 (segment (start 164.445 86.905) (end 164.445 95.865) (width 0.25) (layer "F.Cu") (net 46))
 (segment (start 166.985 95.865) (end 168.58 97.46) (width 0.25) (layer "F.Cu") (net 47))
 (segment (start 166.985 86.905) (end 166.985 95.865) (width 0.25) (layer "F.Cu") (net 47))
 (segment (start 108.825 72.905) (end 120.73 61) (width 0.25) (layer "F.Cu") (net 63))
 (segment (start 139.116 50.884) (end 139.116 49.2) (width 0.25) (layer "F.Cu") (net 63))
 (segment (start 129 61) (end 139.116 50.884) (width 0.25) (layer "F.Cu") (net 63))
 (segment (start 120.73 61) (end 125 61) (width 0.25) (layer "F.Cu") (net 63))
 (via (at 129 61) (size 0.8) (drill 0.4) (layers "F.Cu" "B.Cu") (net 63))
 (via (at 125 61) (size 0.8) (drill 0.4) (layers "F.Cu" "B.Cu") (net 63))
 (segment (start 128 61) (end 129 61) (width 0.25) (layer "B.Cu") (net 63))
 (segment (start 125 61) (end 128 61) (width 0.25) (layer "B.Cu") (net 63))
 (segment (start 121 63) (end 124 63) (width 0.25) (layer "F.Cu") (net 64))
 (segment (start 111.365 72.635) (end 121 63) (width 0.25) (layer "F.Cu") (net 64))
 (segment (start 124 63) (end 125 63) (width 0.25) (layer "F.Cu") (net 64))
 (segment (start 129 63) (end 141.656 50.344) (width 0.25) (layer "F.Cu") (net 64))
 (segment (start 111.365 72.905) (end 111.365 72.635) (width 0.25) (layer "F.Cu") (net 64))
 (segment (start 141.656 50.344) (end 141.656 49.2) (width 0.25) (layer "F.Cu") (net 64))
 (via (at 129 63) (size 0.8) (drill 0.4) (layers "F.Cu" "B.Cu") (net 64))
 (via (at 125 63) (size 0.8) (drill 0.4) (layers "F.Cu" "B.Cu") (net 64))
 (segment (start 125 63) (end 129 63) (width 0.25) (layer "B.Cu") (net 64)))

